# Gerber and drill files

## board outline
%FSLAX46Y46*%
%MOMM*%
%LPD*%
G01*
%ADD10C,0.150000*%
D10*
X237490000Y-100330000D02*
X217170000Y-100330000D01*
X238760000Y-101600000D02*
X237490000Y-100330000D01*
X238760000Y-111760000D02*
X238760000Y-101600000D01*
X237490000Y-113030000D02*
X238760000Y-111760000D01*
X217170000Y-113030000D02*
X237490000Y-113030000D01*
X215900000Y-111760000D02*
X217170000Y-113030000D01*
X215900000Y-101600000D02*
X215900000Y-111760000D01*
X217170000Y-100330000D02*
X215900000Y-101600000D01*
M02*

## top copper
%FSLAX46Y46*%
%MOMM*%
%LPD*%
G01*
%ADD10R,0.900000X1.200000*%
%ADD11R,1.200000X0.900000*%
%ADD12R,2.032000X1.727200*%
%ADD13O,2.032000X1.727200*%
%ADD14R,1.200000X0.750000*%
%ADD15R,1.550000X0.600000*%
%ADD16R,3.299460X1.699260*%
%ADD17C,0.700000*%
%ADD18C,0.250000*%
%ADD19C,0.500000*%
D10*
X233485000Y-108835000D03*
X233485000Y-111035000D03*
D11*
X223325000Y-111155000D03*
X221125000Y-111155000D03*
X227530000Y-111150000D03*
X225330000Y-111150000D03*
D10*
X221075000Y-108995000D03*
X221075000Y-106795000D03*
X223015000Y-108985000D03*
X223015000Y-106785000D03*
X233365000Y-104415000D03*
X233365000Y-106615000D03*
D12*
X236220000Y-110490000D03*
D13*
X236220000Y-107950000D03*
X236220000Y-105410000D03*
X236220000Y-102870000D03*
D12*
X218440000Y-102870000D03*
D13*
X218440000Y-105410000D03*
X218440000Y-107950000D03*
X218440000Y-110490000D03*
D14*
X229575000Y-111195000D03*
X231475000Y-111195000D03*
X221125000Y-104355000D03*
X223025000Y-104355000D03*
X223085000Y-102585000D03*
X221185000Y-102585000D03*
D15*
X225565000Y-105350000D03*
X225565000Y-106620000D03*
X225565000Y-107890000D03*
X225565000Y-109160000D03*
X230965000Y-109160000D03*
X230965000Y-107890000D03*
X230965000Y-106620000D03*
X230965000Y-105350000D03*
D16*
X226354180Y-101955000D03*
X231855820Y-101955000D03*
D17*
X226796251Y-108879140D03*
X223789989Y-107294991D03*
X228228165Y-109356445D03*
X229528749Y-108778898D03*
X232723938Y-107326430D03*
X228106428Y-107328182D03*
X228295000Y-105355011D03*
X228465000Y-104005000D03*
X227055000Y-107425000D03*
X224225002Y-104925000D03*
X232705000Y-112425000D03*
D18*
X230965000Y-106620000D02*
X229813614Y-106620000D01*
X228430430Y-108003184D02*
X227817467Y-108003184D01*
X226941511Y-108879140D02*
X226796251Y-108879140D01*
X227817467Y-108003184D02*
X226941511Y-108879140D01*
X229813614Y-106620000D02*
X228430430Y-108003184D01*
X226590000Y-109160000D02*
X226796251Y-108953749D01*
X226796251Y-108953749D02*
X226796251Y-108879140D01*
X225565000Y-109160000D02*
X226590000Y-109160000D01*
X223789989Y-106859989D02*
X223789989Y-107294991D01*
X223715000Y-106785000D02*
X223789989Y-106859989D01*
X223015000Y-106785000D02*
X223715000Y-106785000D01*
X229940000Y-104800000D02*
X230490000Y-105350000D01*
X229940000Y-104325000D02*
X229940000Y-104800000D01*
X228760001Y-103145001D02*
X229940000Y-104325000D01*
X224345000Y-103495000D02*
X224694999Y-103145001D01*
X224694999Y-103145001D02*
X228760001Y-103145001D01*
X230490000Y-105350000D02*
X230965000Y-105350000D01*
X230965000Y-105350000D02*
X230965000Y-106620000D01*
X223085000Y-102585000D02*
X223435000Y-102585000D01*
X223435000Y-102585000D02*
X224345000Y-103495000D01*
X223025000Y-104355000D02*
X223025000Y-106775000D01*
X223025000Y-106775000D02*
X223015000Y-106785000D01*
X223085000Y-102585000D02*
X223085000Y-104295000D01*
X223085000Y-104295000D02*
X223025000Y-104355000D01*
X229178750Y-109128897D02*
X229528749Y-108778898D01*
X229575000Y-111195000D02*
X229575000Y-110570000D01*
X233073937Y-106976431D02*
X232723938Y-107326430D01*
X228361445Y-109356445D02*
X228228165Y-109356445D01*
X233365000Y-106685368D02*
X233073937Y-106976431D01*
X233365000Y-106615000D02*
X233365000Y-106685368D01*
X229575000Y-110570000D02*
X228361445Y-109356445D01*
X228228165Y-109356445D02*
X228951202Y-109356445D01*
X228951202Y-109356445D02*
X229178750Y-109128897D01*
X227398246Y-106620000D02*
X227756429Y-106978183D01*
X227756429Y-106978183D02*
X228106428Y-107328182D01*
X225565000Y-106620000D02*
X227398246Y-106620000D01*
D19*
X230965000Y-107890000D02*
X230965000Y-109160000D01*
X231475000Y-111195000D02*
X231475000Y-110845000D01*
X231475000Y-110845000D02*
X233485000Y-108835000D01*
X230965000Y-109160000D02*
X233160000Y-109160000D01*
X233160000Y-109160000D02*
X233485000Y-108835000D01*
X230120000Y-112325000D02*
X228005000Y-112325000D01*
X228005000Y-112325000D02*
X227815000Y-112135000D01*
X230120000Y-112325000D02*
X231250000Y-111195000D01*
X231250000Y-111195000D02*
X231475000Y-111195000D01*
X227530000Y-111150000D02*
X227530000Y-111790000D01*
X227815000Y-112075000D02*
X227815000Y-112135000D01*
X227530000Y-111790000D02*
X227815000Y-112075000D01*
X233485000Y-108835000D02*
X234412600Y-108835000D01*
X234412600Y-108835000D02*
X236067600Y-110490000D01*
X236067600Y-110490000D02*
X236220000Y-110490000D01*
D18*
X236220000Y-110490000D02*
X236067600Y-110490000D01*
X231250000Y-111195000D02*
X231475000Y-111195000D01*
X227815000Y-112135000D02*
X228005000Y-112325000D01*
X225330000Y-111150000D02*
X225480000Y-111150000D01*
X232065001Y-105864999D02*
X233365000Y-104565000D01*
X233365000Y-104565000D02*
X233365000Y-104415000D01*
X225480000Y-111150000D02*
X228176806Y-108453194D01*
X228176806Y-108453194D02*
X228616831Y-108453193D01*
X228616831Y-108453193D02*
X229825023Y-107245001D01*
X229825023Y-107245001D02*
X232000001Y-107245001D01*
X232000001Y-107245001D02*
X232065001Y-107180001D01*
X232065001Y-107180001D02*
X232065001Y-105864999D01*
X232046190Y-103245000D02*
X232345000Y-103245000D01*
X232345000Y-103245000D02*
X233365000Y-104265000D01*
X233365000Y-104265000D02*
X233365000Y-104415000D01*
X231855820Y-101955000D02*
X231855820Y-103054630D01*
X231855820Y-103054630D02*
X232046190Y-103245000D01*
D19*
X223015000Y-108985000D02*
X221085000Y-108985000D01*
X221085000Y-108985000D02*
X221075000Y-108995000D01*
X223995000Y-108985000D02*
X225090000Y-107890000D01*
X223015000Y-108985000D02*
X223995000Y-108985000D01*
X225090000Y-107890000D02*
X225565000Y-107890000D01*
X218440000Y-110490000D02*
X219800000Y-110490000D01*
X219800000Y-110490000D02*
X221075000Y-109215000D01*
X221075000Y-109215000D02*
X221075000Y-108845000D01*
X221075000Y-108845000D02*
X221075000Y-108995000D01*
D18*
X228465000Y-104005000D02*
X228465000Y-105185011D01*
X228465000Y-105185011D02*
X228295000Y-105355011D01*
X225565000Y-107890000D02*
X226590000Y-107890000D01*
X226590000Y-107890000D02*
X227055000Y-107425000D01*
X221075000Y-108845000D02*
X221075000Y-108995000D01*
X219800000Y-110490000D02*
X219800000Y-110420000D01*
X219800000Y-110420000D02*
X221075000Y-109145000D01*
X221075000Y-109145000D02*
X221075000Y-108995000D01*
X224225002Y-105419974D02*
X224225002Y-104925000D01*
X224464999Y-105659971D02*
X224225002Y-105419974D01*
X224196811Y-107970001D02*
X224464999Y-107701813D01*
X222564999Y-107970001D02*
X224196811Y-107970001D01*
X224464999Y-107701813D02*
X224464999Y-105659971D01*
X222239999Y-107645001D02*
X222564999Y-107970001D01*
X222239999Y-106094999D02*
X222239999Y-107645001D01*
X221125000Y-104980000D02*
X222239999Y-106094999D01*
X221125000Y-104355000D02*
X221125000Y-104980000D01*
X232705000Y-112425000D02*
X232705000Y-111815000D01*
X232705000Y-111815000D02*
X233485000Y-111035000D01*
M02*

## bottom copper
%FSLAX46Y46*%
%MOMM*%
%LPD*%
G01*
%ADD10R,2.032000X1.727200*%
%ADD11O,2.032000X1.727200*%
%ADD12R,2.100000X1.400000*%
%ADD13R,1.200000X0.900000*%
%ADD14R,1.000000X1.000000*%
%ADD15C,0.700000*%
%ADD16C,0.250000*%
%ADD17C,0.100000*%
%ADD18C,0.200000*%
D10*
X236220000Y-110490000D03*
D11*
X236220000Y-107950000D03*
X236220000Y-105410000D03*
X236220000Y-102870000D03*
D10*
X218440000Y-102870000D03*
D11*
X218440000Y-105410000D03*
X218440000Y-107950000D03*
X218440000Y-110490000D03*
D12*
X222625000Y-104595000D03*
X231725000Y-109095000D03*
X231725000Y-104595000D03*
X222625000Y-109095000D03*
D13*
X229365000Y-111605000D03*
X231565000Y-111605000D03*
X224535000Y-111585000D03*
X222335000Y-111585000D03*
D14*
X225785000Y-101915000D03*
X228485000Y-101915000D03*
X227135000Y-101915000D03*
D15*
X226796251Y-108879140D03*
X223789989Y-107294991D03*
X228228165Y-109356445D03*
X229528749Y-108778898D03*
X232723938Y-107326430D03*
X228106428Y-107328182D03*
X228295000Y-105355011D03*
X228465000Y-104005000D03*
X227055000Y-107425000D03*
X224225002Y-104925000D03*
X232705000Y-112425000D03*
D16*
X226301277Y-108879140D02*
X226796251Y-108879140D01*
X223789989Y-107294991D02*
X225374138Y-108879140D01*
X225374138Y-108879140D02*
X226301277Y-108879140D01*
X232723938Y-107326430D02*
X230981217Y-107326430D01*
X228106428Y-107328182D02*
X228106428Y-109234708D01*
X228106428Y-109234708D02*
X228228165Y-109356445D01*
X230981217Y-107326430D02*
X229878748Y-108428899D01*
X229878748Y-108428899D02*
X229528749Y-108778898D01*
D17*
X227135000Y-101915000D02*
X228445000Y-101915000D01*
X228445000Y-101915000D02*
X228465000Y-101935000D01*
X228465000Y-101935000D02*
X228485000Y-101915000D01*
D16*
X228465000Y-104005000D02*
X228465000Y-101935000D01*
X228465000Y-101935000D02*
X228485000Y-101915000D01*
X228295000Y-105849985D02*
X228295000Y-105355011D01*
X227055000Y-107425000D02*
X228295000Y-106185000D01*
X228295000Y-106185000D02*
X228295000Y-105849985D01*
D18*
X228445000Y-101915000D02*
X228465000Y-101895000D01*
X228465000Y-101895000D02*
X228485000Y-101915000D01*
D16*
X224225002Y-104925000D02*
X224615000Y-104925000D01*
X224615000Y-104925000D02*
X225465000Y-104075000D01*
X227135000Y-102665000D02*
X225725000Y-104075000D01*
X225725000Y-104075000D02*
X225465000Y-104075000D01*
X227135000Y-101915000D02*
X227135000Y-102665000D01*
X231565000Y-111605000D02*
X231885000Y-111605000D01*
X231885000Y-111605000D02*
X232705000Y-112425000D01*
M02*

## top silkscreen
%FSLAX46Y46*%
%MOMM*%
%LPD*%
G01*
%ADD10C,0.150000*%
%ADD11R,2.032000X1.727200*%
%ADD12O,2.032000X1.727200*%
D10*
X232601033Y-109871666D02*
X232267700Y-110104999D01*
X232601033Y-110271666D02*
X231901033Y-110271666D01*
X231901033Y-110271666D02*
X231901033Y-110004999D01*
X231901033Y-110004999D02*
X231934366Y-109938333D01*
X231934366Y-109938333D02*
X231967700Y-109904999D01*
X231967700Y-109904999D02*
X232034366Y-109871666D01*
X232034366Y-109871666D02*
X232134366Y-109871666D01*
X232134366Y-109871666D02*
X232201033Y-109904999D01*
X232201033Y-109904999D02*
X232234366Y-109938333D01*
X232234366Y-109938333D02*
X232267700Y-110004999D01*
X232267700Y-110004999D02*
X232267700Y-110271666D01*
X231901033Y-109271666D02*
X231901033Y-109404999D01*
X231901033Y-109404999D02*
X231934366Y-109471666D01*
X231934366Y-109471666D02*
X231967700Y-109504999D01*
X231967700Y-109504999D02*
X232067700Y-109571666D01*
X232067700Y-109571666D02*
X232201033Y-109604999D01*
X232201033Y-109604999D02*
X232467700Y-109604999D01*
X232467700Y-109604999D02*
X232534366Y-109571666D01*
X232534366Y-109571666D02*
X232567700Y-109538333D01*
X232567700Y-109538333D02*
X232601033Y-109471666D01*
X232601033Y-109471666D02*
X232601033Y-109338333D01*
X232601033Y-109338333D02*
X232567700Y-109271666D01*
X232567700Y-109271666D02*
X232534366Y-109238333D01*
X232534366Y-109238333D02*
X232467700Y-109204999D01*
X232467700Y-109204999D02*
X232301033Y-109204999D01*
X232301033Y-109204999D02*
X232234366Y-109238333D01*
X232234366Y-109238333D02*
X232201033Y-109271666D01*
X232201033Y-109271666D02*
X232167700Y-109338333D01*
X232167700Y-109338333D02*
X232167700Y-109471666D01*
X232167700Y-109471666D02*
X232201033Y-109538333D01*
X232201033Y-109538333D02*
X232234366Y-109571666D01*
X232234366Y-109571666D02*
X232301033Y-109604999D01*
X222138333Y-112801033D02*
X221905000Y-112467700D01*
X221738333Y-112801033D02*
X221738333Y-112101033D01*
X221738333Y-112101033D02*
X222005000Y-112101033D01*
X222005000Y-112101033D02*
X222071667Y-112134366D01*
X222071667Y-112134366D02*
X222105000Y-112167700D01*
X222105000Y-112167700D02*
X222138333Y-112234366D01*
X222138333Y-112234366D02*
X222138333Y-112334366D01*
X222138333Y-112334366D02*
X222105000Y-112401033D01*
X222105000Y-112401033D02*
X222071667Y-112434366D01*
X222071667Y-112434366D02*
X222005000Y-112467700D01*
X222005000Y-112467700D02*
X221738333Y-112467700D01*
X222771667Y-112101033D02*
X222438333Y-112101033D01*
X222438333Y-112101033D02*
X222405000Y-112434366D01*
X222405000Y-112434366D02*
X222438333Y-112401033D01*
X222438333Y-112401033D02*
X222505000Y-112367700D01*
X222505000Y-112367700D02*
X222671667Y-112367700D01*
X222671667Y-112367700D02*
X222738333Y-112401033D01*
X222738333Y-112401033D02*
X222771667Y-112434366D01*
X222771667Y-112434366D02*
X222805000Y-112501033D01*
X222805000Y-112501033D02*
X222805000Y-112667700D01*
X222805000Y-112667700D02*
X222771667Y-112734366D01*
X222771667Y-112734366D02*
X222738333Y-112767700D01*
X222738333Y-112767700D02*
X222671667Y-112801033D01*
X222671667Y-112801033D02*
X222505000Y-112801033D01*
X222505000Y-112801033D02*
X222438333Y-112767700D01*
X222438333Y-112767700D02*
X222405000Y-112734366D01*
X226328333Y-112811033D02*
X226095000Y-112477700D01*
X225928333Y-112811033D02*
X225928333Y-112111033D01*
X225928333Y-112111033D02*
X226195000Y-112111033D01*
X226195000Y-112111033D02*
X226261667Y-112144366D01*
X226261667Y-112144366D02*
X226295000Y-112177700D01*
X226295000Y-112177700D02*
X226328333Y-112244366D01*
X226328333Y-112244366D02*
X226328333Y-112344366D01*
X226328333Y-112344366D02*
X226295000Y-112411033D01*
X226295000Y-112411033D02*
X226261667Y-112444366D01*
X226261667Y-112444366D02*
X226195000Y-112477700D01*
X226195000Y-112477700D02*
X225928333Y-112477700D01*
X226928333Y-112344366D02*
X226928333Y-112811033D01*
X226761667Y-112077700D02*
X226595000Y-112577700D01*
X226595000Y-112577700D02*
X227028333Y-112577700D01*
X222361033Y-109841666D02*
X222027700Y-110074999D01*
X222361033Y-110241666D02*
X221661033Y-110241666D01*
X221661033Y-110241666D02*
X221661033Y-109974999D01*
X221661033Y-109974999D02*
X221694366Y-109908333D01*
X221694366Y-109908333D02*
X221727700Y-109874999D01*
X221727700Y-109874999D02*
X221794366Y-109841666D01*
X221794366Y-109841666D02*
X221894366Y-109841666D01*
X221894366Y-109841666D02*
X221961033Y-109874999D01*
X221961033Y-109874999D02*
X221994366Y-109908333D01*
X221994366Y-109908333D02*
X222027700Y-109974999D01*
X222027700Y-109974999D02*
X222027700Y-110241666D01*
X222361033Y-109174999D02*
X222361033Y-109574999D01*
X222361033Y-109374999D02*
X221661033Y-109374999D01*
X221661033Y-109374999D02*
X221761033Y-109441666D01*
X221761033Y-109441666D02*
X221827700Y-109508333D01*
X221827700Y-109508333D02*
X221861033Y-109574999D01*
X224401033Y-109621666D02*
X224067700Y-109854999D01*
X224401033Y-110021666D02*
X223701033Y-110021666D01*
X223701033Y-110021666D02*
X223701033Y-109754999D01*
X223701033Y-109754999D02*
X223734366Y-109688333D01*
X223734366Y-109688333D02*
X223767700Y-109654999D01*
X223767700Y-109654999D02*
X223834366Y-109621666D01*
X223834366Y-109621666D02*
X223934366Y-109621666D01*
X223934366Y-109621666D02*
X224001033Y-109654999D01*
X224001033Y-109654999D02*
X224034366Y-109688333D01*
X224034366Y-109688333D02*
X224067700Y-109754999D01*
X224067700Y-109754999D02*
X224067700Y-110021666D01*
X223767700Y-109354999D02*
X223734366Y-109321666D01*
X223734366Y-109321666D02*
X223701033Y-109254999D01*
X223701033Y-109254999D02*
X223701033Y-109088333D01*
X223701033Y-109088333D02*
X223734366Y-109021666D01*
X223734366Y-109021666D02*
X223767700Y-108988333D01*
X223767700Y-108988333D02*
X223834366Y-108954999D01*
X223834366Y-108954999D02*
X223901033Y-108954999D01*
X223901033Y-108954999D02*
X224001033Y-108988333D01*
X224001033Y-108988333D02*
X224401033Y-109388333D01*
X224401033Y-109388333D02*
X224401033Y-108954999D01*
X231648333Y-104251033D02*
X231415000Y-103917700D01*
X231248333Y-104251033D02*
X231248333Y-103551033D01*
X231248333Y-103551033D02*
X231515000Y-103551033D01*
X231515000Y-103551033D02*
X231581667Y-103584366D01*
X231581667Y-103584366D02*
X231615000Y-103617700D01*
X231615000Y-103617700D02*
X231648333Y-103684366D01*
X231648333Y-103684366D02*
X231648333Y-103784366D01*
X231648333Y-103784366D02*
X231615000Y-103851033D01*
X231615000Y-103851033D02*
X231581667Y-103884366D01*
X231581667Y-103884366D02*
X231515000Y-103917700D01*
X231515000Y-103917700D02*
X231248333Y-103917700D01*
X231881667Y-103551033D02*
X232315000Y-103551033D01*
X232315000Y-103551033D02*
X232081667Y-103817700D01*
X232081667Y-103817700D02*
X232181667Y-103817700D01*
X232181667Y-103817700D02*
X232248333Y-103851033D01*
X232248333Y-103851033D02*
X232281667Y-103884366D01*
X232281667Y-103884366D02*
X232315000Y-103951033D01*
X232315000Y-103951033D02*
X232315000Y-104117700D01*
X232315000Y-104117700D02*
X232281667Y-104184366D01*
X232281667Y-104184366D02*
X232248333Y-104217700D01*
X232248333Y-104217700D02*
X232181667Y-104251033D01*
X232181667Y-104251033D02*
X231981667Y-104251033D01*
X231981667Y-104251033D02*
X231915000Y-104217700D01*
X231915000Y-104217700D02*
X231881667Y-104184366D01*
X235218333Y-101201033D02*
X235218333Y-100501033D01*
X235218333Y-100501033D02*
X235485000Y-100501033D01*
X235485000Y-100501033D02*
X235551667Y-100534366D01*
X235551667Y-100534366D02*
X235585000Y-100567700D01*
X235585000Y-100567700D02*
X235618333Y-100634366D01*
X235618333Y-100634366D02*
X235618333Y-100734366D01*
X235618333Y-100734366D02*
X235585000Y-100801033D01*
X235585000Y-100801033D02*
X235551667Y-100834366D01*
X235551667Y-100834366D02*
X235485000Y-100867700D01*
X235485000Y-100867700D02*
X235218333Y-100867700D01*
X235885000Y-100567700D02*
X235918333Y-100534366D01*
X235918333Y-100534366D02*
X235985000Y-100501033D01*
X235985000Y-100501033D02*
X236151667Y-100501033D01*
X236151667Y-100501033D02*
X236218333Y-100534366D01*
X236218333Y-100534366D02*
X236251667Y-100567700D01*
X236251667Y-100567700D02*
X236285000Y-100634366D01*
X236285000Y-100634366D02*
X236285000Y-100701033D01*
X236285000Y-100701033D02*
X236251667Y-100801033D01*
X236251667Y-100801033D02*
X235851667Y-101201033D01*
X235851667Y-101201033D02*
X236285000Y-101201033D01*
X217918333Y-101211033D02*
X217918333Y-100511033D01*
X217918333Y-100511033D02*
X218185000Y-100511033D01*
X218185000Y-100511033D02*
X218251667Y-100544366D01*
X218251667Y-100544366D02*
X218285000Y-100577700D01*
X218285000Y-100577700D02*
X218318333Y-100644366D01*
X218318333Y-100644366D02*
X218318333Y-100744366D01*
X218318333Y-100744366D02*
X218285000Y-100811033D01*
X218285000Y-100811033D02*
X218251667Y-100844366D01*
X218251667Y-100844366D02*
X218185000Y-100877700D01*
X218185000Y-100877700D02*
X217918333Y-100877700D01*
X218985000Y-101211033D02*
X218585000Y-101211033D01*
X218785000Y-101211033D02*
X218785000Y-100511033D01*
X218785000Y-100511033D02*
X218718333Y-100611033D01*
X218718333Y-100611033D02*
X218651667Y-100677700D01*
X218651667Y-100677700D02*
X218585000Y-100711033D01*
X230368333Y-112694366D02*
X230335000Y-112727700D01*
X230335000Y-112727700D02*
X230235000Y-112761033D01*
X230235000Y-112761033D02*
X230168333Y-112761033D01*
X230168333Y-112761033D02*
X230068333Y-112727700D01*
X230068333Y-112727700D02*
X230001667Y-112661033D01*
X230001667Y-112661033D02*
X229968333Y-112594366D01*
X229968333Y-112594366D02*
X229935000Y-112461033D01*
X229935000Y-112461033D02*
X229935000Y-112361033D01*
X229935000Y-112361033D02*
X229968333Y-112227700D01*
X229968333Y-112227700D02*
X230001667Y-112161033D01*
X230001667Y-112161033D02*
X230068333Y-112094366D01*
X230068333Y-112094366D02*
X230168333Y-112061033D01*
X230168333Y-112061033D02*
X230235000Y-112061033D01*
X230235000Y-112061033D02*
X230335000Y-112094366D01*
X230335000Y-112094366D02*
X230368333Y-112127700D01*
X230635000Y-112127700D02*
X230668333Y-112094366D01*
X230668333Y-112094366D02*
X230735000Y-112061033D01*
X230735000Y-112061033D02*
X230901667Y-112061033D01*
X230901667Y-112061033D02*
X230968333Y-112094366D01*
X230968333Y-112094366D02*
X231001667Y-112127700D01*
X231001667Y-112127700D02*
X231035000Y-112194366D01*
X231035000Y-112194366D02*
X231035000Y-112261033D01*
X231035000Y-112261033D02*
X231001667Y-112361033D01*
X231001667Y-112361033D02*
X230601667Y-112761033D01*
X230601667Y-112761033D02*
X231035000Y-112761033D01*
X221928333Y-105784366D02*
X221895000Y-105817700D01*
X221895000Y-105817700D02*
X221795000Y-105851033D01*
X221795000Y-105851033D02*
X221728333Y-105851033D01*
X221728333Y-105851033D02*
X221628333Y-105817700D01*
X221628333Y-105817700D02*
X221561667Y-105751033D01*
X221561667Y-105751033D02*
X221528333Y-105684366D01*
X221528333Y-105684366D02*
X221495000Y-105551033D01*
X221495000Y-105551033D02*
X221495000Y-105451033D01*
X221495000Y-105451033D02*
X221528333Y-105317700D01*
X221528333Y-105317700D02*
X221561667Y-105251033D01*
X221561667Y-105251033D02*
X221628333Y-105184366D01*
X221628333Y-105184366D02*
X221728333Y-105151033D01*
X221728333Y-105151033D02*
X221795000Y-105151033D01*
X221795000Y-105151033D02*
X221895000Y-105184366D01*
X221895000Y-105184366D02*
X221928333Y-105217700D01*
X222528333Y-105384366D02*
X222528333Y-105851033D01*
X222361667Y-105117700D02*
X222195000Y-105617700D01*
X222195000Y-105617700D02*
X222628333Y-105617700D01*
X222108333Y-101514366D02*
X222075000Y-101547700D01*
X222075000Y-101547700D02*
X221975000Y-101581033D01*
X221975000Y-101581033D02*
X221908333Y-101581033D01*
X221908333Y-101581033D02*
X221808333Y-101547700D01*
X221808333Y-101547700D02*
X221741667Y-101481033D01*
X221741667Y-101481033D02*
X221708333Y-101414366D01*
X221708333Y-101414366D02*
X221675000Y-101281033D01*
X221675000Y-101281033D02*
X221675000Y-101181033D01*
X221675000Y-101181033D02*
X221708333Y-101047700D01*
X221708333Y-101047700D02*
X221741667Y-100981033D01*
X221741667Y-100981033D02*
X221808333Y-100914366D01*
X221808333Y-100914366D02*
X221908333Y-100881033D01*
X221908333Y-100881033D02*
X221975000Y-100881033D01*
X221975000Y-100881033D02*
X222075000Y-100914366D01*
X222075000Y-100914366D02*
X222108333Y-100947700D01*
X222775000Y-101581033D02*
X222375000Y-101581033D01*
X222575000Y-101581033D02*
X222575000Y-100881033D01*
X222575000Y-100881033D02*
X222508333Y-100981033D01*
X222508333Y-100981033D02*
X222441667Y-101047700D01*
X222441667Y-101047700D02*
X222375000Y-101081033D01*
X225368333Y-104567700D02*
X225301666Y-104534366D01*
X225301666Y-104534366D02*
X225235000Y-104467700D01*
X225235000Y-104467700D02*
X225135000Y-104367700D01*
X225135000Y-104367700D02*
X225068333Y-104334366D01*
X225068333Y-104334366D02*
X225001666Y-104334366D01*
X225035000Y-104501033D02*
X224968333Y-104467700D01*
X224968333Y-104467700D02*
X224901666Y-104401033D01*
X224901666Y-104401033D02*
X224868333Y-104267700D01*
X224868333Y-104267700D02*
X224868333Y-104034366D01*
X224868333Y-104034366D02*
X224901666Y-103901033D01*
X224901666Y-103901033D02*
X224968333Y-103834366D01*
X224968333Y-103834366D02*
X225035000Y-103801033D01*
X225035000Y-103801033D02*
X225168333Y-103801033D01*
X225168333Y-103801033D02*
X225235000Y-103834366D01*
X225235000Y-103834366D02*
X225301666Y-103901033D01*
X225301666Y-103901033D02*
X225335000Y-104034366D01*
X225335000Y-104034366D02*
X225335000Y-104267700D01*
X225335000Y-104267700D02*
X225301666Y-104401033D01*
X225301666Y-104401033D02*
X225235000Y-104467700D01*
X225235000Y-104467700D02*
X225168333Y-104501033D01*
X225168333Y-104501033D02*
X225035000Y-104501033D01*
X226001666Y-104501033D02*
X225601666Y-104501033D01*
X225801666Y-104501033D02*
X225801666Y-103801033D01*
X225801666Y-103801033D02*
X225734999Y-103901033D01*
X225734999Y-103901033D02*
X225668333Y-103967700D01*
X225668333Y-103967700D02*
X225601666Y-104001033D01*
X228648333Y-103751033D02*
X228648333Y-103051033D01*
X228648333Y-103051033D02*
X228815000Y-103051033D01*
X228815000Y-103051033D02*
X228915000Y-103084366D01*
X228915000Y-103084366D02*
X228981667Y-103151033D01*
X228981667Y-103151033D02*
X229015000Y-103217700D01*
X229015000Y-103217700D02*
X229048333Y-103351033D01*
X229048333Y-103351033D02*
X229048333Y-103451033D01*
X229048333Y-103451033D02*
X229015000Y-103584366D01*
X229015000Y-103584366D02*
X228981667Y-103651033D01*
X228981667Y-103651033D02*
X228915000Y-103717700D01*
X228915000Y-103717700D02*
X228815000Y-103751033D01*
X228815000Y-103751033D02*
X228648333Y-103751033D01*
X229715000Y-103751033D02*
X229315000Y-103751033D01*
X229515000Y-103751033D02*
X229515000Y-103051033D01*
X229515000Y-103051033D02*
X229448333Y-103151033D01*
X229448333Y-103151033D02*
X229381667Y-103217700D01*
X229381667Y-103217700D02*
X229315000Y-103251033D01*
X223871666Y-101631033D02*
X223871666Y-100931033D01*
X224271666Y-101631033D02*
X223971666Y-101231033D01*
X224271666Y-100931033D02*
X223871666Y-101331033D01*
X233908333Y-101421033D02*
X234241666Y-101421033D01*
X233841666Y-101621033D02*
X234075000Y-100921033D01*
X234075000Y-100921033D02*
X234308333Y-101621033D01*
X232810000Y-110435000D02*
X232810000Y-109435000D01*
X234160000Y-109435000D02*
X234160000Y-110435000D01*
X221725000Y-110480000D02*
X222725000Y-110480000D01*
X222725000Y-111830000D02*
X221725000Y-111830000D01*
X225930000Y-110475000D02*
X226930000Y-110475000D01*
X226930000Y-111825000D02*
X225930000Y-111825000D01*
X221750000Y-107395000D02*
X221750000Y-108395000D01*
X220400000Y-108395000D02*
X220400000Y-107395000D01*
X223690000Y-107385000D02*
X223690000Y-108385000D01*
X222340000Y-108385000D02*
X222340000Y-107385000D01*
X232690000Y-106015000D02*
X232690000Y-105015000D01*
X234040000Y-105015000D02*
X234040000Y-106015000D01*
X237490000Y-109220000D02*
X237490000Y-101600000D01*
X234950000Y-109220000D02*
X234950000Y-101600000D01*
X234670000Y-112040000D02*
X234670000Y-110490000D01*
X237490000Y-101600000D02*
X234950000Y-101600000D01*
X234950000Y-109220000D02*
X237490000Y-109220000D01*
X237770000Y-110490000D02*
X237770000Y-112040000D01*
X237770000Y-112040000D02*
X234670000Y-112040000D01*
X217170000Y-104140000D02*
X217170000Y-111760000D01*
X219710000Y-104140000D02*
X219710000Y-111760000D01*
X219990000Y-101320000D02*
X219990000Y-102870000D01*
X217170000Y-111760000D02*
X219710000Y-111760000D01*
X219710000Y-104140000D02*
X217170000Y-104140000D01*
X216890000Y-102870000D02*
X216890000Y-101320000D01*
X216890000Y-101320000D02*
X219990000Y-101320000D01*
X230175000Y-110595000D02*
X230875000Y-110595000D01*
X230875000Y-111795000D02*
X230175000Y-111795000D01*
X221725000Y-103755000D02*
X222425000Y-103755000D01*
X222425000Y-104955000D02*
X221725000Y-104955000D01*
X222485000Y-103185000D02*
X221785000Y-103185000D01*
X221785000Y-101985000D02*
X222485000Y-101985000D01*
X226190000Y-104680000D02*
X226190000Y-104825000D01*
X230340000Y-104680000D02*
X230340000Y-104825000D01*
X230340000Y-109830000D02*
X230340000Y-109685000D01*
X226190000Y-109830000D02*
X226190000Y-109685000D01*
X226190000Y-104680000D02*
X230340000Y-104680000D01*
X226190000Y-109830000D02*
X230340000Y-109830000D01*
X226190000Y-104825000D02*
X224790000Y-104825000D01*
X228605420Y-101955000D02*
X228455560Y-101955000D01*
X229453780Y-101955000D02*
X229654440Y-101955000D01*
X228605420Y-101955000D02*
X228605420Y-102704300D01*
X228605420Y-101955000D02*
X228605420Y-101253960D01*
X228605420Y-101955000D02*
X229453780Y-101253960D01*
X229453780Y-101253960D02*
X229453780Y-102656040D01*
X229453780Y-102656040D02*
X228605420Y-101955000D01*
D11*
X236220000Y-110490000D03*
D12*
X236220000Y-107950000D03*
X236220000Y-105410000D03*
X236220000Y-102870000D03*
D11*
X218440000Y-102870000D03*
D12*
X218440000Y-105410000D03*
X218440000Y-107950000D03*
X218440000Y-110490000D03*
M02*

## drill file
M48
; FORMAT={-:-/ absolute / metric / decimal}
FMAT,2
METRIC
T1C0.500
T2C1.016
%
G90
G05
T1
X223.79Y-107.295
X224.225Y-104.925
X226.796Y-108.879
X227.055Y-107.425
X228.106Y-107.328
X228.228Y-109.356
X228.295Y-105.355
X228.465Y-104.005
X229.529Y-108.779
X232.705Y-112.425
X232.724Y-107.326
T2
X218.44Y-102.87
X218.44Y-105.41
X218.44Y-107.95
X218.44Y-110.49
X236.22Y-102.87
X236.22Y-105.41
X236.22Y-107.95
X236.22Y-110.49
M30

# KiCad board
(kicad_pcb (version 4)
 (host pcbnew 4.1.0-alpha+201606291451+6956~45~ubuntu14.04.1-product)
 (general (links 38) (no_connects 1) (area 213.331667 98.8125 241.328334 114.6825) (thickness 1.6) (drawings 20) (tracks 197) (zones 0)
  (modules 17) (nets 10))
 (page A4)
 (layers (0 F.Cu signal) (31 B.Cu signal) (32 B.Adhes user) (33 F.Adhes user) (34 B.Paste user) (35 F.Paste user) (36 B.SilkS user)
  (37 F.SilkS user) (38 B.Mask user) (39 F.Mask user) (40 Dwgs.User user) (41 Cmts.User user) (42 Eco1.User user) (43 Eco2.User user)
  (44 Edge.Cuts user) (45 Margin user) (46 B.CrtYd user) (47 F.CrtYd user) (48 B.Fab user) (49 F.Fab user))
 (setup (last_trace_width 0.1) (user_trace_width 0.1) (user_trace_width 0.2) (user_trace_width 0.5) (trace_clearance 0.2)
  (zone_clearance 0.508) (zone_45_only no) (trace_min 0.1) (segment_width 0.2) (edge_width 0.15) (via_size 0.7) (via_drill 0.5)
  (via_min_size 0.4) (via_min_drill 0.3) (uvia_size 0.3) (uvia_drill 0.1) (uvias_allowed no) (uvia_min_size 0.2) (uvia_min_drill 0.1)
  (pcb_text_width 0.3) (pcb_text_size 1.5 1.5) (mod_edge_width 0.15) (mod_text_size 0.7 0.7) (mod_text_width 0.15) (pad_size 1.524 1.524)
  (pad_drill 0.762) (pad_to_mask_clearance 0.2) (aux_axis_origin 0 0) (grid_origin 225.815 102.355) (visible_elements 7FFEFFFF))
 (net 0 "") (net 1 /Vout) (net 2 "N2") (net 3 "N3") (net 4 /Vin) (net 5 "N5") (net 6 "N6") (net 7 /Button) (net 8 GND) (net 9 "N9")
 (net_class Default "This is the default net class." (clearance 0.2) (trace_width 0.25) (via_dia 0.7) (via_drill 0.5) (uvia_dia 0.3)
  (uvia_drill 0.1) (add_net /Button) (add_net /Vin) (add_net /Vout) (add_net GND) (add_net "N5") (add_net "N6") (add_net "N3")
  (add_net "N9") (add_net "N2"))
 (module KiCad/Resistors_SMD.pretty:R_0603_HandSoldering (layer F.Cu) (at 233.485 109.935 270)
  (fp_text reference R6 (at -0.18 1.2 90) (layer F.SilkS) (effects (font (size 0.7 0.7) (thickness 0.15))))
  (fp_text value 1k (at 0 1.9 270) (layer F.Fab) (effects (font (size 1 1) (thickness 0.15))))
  (fp_line (start 0.5 0.675) (end -0.5 0.675) (layer F.SilkS) (width 0.15))
  (fp_line (start -0.5 -0.675) (end 0.5 -0.675) (layer F.SilkS) (width 0.15))
  (pad 1 smd rect (at -1.1 0 270) (size 1.2 0.9) (layers F.Cu F.Paste F.Mask) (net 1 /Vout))
  (pad 2 smd rect (at 1.1 0 270) (size 1.2 0.9) (layers F.Cu F.Paste F.Mask) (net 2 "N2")))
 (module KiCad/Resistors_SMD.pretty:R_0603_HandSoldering (layer F.Cu) (at 222.225 111.155 180)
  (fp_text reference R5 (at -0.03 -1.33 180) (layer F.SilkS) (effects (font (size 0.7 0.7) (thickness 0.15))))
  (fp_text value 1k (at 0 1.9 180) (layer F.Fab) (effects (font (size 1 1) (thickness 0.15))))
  (fp_line (start 0.5 0.675) (end -0.5 0.675) (layer F.SilkS) (width 0.15))
  (fp_line (start -0.5 -0.675) (end 0.5 -0.675) (layer F.SilkS) (width 0.15))
  (pad 1 smd rect (at -1.1 0 180) (size 1.2 0.9) (layers F.Cu F.Paste F.Mask))
  (pad 2 smd rect (at 1.1 0 180) (size 1.2 0.9) (layers F.Cu F.Paste F.Mask)))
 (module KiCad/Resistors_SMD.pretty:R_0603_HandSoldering (layer F.Cu) (at 226.43 111.15 180)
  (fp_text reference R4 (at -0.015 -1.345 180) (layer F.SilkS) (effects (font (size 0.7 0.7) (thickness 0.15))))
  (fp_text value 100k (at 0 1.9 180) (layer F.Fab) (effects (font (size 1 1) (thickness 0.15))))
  (fp_line (start 0.5 0.675) (end -0.5 0.675) (layer F.SilkS) (width 0.15))
  (fp_line (start -0.5 -0.675) (end 0.5 -0.675) (layer F.SilkS) (width 0.15))
  (pad 1 smd rect (at -1.1 0 180) (size 1.2 0.9) (layers F.Cu F.Paste F.Mask) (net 1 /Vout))
  (pad 2 smd rect (at 1.1 0 180) (size 1.2 0.9) (layers F.Cu F.Paste F.Mask) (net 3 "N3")))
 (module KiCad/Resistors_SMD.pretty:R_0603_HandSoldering (layer F.Cu) (at 221.075 107.895 90)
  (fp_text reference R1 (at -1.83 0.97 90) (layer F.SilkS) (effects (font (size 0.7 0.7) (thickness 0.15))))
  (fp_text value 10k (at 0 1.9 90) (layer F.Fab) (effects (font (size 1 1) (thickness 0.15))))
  (fp_line (start 0.5 0.675) (end -0.5 0.675) (layer F.SilkS) (width 0.15))
  (fp_line (start -0.5 -0.675) (end 0.5 -0.675) (layer F.SilkS) (width 0.15))
  (pad 1 smd rect (at -1.1 0 90) (size 1.2 0.9) (layers F.Cu F.Paste F.Mask) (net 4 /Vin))
  (pad 2 smd rect (at 1.1 0 90) (size 1.2 0.9) (layers F.Cu F.Paste F.Mask)))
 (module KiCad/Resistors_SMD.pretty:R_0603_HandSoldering (layer F.Cu) (at 223.015 107.885 90)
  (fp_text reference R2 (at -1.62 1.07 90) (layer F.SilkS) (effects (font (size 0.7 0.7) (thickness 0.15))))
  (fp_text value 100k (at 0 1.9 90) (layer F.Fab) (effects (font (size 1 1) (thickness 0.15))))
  (fp_line (start 0.5 0.675) (end -0.5 0.675) (layer F.SilkS) (width 0.15))
  (fp_line (start -0.5 -0.675) (end 0.5 -0.675) (layer F.SilkS) (width 0.15))
  (pad 1 smd rect (at -1.1 0 90) (size 1.2 0.9) (layers F.Cu F.Paste F.Mask) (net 4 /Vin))
  (pad 2 smd rect (at 1.1 0 90) (size 1.2 0.9) (layers F.Cu F.Paste F.Mask) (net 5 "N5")))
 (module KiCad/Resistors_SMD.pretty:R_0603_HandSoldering (layer F.Cu) (at 233.365 105.515 270)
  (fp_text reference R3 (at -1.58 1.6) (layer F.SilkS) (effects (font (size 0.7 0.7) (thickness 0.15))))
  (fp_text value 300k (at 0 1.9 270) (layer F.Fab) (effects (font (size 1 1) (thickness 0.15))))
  (fp_line (start 0.5 0.675) (end -0.5 0.675) (layer F.SilkS) (width 0.15))
  (fp_line (start -0.5 -0.675) (end 0.5 -0.675) (layer F.SilkS) (width 0.15))
  (pad 1 smd rect (at -1.1 0 270) (size 1.2 0.9) (layers F.Cu F.Paste F.Mask) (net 3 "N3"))
  (pad 2 smd rect (at 1.1 0 270) (size 1.2 0.9) (layers F.Cu F.Paste F.Mask) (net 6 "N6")))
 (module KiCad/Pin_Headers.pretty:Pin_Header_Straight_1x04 (layer F.Cu) (at 236.22 110.49 180)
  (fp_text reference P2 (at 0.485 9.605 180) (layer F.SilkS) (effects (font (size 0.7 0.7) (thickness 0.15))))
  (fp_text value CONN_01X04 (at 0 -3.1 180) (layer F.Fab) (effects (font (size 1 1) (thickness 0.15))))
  (fp_line (start -1.27 1.27) (end -1.27 8.89) (layer F.SilkS) (width 0.15))
  (fp_line (start 1.27 1.27) (end 1.27 8.89) (layer F.SilkS) (width 0.15))
  (fp_line (start 1.55 -1.55) (end 1.55 0) (layer F.SilkS) (width 0.15))
  (fp_line (start -1.27 8.89) (end 1.27 8.89) (layer F.SilkS) (width 0.15))
  (fp_line (start 1.27 1.27) (end -1.27 1.27) (layer F.SilkS) (width 0.15))
  (fp_line (start -1.55 0) (end -1.55 -1.55) (layer F.SilkS) (width 0.15))
  (fp_line (start -1.55 -1.55) (end 1.55 -1.55) (layer F.SilkS) (width 0.15))
  (pad 1 thru_hole rect (at 0 0 180) (size 2.032 1.7272) (drill 1.016) (layers *.Cu *.Mask F.SilkS) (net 1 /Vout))
  (pad 2 thru_hole oval (at 0 2.54 180) (size 2.032 1.7272) (drill 1.016) (layers *.Cu *.Mask F.SilkS))
  (pad 3 thru_hole oval (at 0 5.08 180) (size 2.032 1.7272) (drill 1.016) (layers *.Cu *.Mask F.SilkS))
  (pad 4 thru_hole oval (at 0 7.62 180) (size 2.032 1.7272) (drill 1.016) (layers *.Cu *.Mask F.SilkS)))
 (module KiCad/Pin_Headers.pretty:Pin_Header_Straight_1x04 (layer F.Cu) (at 218.44 102.87)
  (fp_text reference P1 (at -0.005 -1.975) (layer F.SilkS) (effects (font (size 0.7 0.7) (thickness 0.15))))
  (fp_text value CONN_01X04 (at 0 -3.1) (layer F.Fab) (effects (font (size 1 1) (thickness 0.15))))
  (fp_line (start -1.27 1.27) (end -1.27 8.89) (layer F.SilkS) (width 0.15))
  (fp_line (start 1.27 1.27) (end 1.27 8.89) (layer F.SilkS) (width 0.15))
  (fp_line (start 1.55 -1.55) (end 1.55 0) (layer F.SilkS) (width 0.15))
  (fp_line (start -1.27 8.89) (end 1.27 8.89) (layer F.SilkS) (width 0.15))
  (fp_line (start 1.27 1.27) (end -1.27 1.27) (layer F.SilkS) (width 0.15))
  (fp_line (start -1.55 0) (end -1.55 -1.55) (layer F.SilkS) (width 0.15))
  (fp_line (start -1.55 -1.55) (end 1.55 -1.55) (layer F.SilkS) (width 0.15))
  (pad 1 thru_hole rect (at 0 0) (size 2.032 1.7272) (drill 1.016) (layers *.Cu *.Mask F.SilkS))
  (pad 2 thru_hole oval (at 0 2.54) (size 2.032 1.7272) (drill 1.016) (layers *.Cu *.Mask F.SilkS))
  (pad 3 thru_hole oval (at 0 5.08) (size 2.032 1.7272) (drill 1.016) (layers *.Cu *.Mask F.SilkS))
  (pad 4 thru_hole oval (at 0 7.62) (size 2.032 1.7272) (drill 1.016) (layers *.Cu *.Mask F.SilkS) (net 4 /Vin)))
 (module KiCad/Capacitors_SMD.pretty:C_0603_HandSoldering (layer F.Cu) (at 230.525 111.195)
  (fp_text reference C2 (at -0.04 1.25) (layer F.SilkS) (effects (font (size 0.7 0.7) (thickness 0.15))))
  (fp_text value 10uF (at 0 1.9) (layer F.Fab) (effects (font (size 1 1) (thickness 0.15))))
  (fp_line (start -0.35 -0.6) (end 0.35 -0.6) (layer F.SilkS) (width 0.15))
  (fp_line (start 0.35 0.6) (end -0.35 0.6) (layer F.SilkS) (width 0.15))
  (pad 1 smd rect (at -0.95 0) (size 1.2 0.75) (layers F.Cu F.Paste F.Mask) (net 6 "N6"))
  (pad 2 smd rect (at 0.95 0) (size 1.2 0.75) (layers F.Cu F.Paste F.Mask) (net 1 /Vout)))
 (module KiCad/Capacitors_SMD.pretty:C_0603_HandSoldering (layer F.Cu) (at 222.075 104.355)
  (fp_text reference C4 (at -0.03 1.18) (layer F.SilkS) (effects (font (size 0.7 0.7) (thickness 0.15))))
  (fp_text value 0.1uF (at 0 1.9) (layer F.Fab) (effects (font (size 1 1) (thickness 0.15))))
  (fp_line (start -0.35 -0.6) (end 0.35 -0.6) (layer F.SilkS) (width 0.15))
  (fp_line (start 0.35 0.6) (end -0.35 0.6) (layer F.SilkS) (width 0.15))
  (pad 1 smd rect (at -0.95 0) (size 1.2 0.75) (layers F.Cu F.Paste F.Mask) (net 4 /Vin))
  (pad 2 smd rect (at 0.95 0) (size 1.2 0.75) (layers F.Cu F.Paste F.Mask) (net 5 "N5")))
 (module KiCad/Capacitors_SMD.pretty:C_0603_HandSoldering (layer F.Cu) (at 222.135 102.585 180)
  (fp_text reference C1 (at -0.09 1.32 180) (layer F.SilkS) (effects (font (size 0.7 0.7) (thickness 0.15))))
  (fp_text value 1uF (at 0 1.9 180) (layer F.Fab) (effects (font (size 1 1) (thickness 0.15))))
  (fp_line (start -0.35 -0.6) (end 0.35 -0.6) (layer F.SilkS) (width 0.15))
  (fp_line (start 0.35 0.6) (end -0.35 0.6) (layer F.SilkS) (width 0.15))
  (pad 1 smd rect (at -0.95 0 180) (size 1.2 0.75) (layers F.Cu F.Paste F.Mask) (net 5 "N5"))
  (pad 2 smd rect (at 0.95 0 180) (size 1.2 0.75) (layers F.Cu F.Paste F.Mask)))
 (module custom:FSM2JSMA (layer B.Cu) (at 227.175 106.845 270)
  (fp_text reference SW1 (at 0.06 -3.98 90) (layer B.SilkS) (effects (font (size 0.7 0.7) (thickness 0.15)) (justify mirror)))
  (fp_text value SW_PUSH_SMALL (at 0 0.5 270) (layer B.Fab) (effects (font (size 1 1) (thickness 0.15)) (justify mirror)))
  (pad 2 smd rect (at -2.25 4.55 270) (size 1.4 2.1) (layers B.Cu B.Paste B.Mask))
  (pad 1 smd rect (at 2.25 -4.55 270) (size 1.4 2.1) (layers B.Cu B.Paste B.Mask))
  (pad 2 smd rect (at -2.25 -4.55 270) (size 1.4 2.1) (layers B.Cu B.Paste B.Mask))
  (pad 1 smd rect (at 2.25 4.55 270) (size 1.4 2.1) (layers B.Cu B.Paste B.Mask)))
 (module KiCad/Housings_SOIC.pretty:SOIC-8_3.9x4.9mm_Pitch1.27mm (layer F.Cu) (at 228.265 107.255)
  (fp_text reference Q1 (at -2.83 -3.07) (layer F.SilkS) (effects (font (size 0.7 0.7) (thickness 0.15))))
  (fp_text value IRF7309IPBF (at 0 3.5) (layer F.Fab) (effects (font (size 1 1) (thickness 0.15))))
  (fp_line (start -2.075 -2.575) (end -2.075 -2.43) (layer F.SilkS) (width 0.15))
  (fp_line (start 2.075 -2.575) (end 2.075 -2.43) (layer F.SilkS) (width 0.15))
  (fp_line (start 2.075 2.575) (end 2.075 2.43) (layer F.SilkS) (width 0.15))
  (fp_line (start -2.075 2.575) (end -2.075 2.43) (layer F.SilkS) (width 0.15))
  (fp_line (start -2.075 -2.575) (end 2.075 -2.575) (layer F.SilkS) (width 0.15))
  (fp_line (start -2.075 2.575) (end 2.075 2.575) (layer F.SilkS) (width 0.15))
  (fp_line (start -2.075 -2.43) (end -3.475 -2.43) (layer F.SilkS) (width 0.15))
  (pad 1 smd rect (at -2.7 -1.905) (size 1.55 0.6) (layers F.Cu F.Paste F.Mask))
  (pad 2 smd rect (at -2.7 -0.635) (size 1.55 0.6) (layers F.Cu F.Paste F.Mask) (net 6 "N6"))
  (pad 3 smd rect (at -2.7 0.635) (size 1.55 0.6) (layers F.Cu F.Paste F.Mask) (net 4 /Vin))
  (pad 4 smd rect (at -2.7 1.905) (size 1.55 0.6) (layers F.Cu F.Paste F.Mask) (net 5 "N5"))
  (pad 5 smd rect (at 2.7 1.905) (size 1.55 0.6) (layers F.Cu F.Paste F.Mask) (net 1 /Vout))
  (pad 6 smd rect (at 2.7 0.635) (size 1.55 0.6) (layers F.Cu F.Paste F.Mask) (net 1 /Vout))
  (pad 7 smd rect (at 2.7 -0.635) (size 1.55 0.6) (layers F.Cu F.Paste F.Mask) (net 5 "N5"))
  (pad 8 smd rect (at 2.7 -1.905) (size 1.55 0.6) (layers F.Cu F.Paste F.Mask) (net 5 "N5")))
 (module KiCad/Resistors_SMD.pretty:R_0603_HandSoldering (layer B.Cu) (at 230.465 111.605)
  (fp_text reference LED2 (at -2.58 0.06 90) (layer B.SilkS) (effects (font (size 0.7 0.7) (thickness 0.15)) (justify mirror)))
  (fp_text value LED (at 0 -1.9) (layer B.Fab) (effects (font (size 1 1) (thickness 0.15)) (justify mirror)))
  (pad 1 smd rect (at -1.1 0) (size 1.2 0.9) (layers B.Cu B.Paste B.Mask))
  (pad 2 smd rect (at 1.1 0) (size 1.2 0.9) (layers B.Cu B.Paste B.Mask) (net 2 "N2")))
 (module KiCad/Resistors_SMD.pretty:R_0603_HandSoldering (layer B.Cu) (at 223.435 111.585 180)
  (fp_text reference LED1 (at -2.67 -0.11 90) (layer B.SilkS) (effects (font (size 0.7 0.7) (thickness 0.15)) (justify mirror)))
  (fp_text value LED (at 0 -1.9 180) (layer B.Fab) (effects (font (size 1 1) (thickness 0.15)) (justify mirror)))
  (pad 1 smd rect (at -1.1 0 180) (size 1.2 0.9) (layers B.Cu B.Paste B.Mask))
  (pad 2 smd rect (at 1.1 0 180) (size 1.2 0.9) (layers B.Cu B.Paste B.Mask)))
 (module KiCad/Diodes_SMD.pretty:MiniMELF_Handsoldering (layer F.Cu) (at 229.105 101.955)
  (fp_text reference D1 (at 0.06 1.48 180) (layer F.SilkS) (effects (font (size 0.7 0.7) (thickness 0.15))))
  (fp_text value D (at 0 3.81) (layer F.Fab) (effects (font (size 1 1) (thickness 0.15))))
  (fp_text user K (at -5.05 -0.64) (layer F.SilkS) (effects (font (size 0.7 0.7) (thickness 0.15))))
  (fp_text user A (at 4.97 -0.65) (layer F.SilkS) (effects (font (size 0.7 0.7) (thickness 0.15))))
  (fp_line (start -0.49958 0) (end -0.64944 0) (layer F.SilkS) (width 0.15))
  (fp_line (start 0.34878 0) (end 0.54944 0) (layer F.SilkS) (width 0.15))
  (fp_line (start -0.49958 0) (end -0.49958 0.7493) (layer F.SilkS) (width 0.15))
  (fp_line (start -0.49958 0) (end -0.49958 -0.70104) (layer F.SilkS) (width 0.15))
  (fp_line (start -0.49958 0) (end 0.34878 -0.70104) (layer F.SilkS) (width 0.15))
  (fp_line (start 0.34878 -0.70104) (end 0.34878 0.70104) (layer F.SilkS) (width 0.15))
  (fp_line (start 0.34878 0.70104) (end -0.49958 0) (layer F.SilkS) (width 0.15))
  (pad 1 smd rect (at -2.75082 0) (size 3.29946 1.69926) (layers F.Cu F.Paste F.Mask))
  (pad 2 smd rect (at 2.75082 0) (size 3.29946 1.69926) (layers F.Cu F.Paste F.Mask) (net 3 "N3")))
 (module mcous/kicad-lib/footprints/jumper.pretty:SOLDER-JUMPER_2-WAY (layer B.Cu) (at 227.135 101.915)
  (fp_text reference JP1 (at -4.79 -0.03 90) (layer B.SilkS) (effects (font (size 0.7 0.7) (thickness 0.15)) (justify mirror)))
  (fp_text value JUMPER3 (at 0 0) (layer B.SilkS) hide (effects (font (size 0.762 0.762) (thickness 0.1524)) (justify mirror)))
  (pad 1 smd rect (at -1.35 0) (size 1 1) (layers B.Cu B.Paste B.Mask))
  (pad 3 smd rect (at 1.35 0) (size 1 1) (layers B.Cu B.Paste B.Mask) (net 4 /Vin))
  (pad 2 smd rect (at 0 0) (size 1 1) (layers B.Cu B.Paste B.Mask) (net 4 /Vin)))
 (gr_line (start 237.49 100.33) (end 217.17 100.33) (angle 90) (layer Edge.Cuts) (width 0.15))
 (gr_line (start 238.76 101.6) (end 237.49 100.33) (angle 90) (layer Edge.Cuts) (width 0.15))
 (gr_line (start 238.76 111.76) (end 238.76 101.6) (angle 90) (layer Edge.Cuts) (width 0.15))
 (gr_line (start 237.49 113.03) (end 238.76 111.76) (angle 90) (layer Edge.Cuts) (width 0.15))
 (gr_line (start 217.17 113.03) (end 237.49 113.03) (angle 90) (layer Edge.Cuts) (width 0.15))
 (gr_line (start 215.9 111.76) (end 217.17 113.03) (angle 90) (layer Edge.Cuts) (width 0.15))
 (gr_line (start 215.9 101.6) (end 215.9 111.76) (angle 90) (layer Edge.Cuts) (width 0.15))
 (gr_line (start 217.17 100.33) (end 215.9 101.6) (angle 90) (layer Edge.Cuts) (width 0.15))
 (segment (start 230.965 106.62) (end 229.813614 106.62) (width 0.25) (layer F.Cu) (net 5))
 (segment (start 228.43043 108.003184) (end 227.817467 108.003184) (width 0.25) (layer F.Cu) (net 5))
 (segment (start 226.941511 108.87914) (end 226.796251 108.87914) (width 0.25) (layer F.Cu) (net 5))
 (segment (start 227.817467 108.003184) (end 226.941511 108.87914) (width 0.25) (layer F.Cu) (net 5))
 (segment (start 226.301277 108.87914) (end 226.796251 108.87914) (width 0.25) (layer B.Cu) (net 5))
 (segment (start 229.813614 106.62) (end 228.43043 108.003184) (width 0.25) (layer F.Cu) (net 5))
 (segment (start 223.789989 107.294991) (end 225.374138 108.87914) (width 0.25) (layer B.Cu) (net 5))
 (segment (start 226.59 109.16) (end 226.796251 108.953749) (width 0.25) (layer F.Cu) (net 5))
 (segment (start 225.374138 108.87914) (end 226.301277 108.87914) (width 0.25) (layer B.Cu) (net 5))
 (segment (start 226.796251 108.953749) (end 226.796251 108.87914) (width 0.25) (layer F.Cu) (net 5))
 (segment (start 225.565 109.16) (end 226.59 109.16) (width 0.25) (layer F.Cu) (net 5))
 (segment (start 223.789989 106.859989) (end 223.789989 107.294991) (width 0.25) (layer F.Cu) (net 5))
 (segment (start 223.715 106.785) (end 223.789989 106.859989) (width 0.25) (layer F.Cu) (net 5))
 (segment (start 223.015 106.785) (end 223.715 106.785) (width 0.25) (layer F.Cu) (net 5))
 (segment (start 229.94 104.8) (end 230.49 105.35) (width 0.25) (layer F.Cu) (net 5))
 (segment (start 229.94 104.325) (end 229.94 104.8) (width 0.25) (layer F.Cu) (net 5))
 (segment (start 228.760001 103.145001) (end 229.94 104.325) (width 0.25) (layer F.Cu) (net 5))
 (segment (start 224.345 103.495) (end 224.694999 103.145001) (width 0.25) (layer F.Cu) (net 5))
 (segment (start 224.694999 103.145001) (end 228.760001 103.145001) (width 0.25) (layer F.Cu) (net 5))
 (segment (start 230.49 105.35) (end 230.965 105.35) (width 0.25) (layer F.Cu) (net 5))
 (segment (start 230.965 105.35) (end 230.965 106.62) (width 0.25) (layer F.Cu) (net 5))
 (segment (start 223.085 102.585) (end 223.435 102.585) (width 0.25) (layer F.Cu) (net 5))
 (segment (start 223.435 102.585) (end 224.345 103.495) (width 0.25) (layer F.Cu) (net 5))
 (segment (start 223.025 104.355) (end 223.025 106.775) (width 0.25) (layer F.Cu) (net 5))
 (segment (start 223.025 106.775) (end 223.015 106.785) (width 0.25) (layer F.Cu) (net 5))
 (segment (start 223.085 102.585) (end 223.085 104.295) (width 0.25) (layer F.Cu) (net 5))
 (segment (start 223.085 104.295) (end 223.025 104.355) (width 0.25) (layer F.Cu) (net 5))
 (segment (start 229.17875 109.128897) (end 229.528749 108.778898) (width 0.25) (layer F.Cu) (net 6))
 (segment (start 229.575 111.195) (end 229.575 110.57) (width 0.25) (layer F.Cu) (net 6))
 (segment (start 233.073937 106.976431) (end 232.723938 107.32643) (width 0.25) (layer F.Cu) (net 6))
 (segment (start 232.723938 107.32643) (end 230.981217 107.32643) (width 0.25) (layer B.Cu) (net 6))
 (segment (start 228.361445 109.356445) (end 228.228165 109.356445) (width 0.25) (layer F.Cu) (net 6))
 (segment (start 233.365 106.685368) (end 233.073937 106.976431) (width 0.25) (layer F.Cu) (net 6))
 (segment (start 228.106428 107.328182) (end 228.106428 109.234708) (width 0.25) (layer B.Cu) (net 6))
 (segment (start 228.106428 109.234708) (end 228.228165 109.356445) (width 0.25) (layer B.Cu) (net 6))
 (segment (start 233.365 106.615) (end 233.365 106.685368) (width 0.25) (layer F.Cu) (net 6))
 (segment (start 229.575 110.57) (end 228.361445 109.356445) (width 0.25) (layer F.Cu) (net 6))
 (segment (start 230.981217 107.32643) (end 229.878748 108.428899) (width 0.25) (layer B.Cu) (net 6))
 (segment (start 229.878748 108.428899) (end 229.528749 108.778898) (width 0.25) (layer B.Cu) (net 6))
 (segment (start 228.228165 109.356445) (end 228.951202 109.356445) (width 0.25) (layer F.Cu) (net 6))
 (segment (start 228.951202 109.356445) (end 229.17875 109.128897) (width 0.25) (layer F.Cu) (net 6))
 (segment (start 227.398246 106.62) (end 227.756429 106.978183) (width 0.25) (layer F.Cu) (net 6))
 (segment (start 227.756429 106.978183) (end 228.106428 107.328182) (width 0.25) (layer F.Cu) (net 6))
 (segment (start 225.565 106.62) (end 227.398246 106.62) (width 0.25) (layer F.Cu) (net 6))
 (segment (start 230.965 107.89) (end 230.965 109.16) (width 0.5) (layer F.Cu) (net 1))
 (segment (start 231.475 111.195) (end 231.475 110.845) (width 0.5) (layer F.Cu) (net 1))
 (segment (start 231.475 110.845) (end 233.485 108.835) (width 0.5) (layer F.Cu) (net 1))
 (segment (start 230.965 109.16) (end 233.16 109.16) (width 0.5) (layer F.Cu) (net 1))
 (segment (start 233.16 109.16) (end 233.485 108.835) (width 0.5) (layer F.Cu) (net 1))
 (segment (start 230.12 112.325) (end 228.005 112.325) (width 0.5) (layer F.Cu) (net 1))
 (segment (start 228.005 112.325) (end 227.815 112.135) (width 0.5) (layer F.Cu) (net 1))
 (segment (start 230.12 112.325) (end 231.25 111.195) (width 0.5) (layer F.Cu) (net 1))
 (segment (start 231.25 111.195) (end 231.475 111.195) (width 0.5) (layer F.Cu) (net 1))
 (segment (start 227.53 111.15) (end 227.53 111.79) (width 0.5) (layer F.Cu) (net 1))
 (segment (start 227.815 112.075) (end 227.815 112.135) (width 0.5) (layer F.Cu) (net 1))
 (segment (start 227.53 111.79) (end 227.815 112.075) (width 0.5) (layer F.Cu) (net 1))
 (segment (start 233.485 108.835) (end 234.4126 108.835) (width 0.5) (layer F.Cu) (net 1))
 (segment (start 234.4126 108.835) (end 236.0676 110.49) (width 0.5) (layer F.Cu) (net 1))
 (segment (start 236.0676 110.49) (end 236.22 110.49) (width 0.5) (layer F.Cu) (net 1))
 (segment (start 236.22 110.49) (end 236.0676 110.49) (width 0.25) (layer F.Cu) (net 1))
 (segment (start 231.25 111.195) (end 231.475 111.195) (width 0.25) (layer F.Cu) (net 1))
 (segment (start 227.815 112.135) (end 228.005 112.325) (width 0.25) (layer F.Cu) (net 1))
 (segment (start 225.33 111.15) (end 225.48 111.15) (width 0.25) (layer F.Cu) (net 3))
 (segment (start 232.065001 105.864999) (end 233.365 104.565) (width 0.25) (layer F.Cu) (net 3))
 (segment (start 233.365 104.565) (end 233.365 104.415) (width 0.25) (layer F.Cu) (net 3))
 (segment (start 225.48 111.15) (end 228.176806 108.453194) (width 0.25) (layer F.Cu) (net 3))
 (segment (start 228.176806 108.453194) (end 228.616831 108.453193) (width 0.25) (layer F.Cu) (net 3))
 (segment (start 228.616831 108.453193) (end 229.825023 107.245001) (width 0.25) (layer F.Cu) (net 3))
 (segment (start 229.825023 107.245001) (end 232.000001 107.245001) (width 0.25) (layer F.Cu) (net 3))
 (segment (start 232.000001 107.245001) (end 232.065001 107.180001) (width 0.25) (layer F.Cu) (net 3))
 (segment (start 232.065001 107.180001) (end 232.065001 105.864999) (width 0.25) (layer F.Cu) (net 3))
 (segment (start 232.04619 103.245) (end 232.345 103.245) (width 0.25) (layer F.Cu) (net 3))
 (segment (start 232.345 103.245) (end 233.365 104.265) (width 0.25) (layer F.Cu) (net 3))
 (segment (start 233.365 104.265) (end 233.365 104.415) (width 0.25) (layer F.Cu) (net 3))
 (segment (start 231.85582 101.955) (end 231.85582 103.05463) (width 0.25) (layer F.Cu) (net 3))
 (segment (start 231.85582 103.05463) (end 232.04619 103.245) (width 0.25) (layer F.Cu) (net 3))
 (segment (start 227.135 101.915) (end 228.445 101.915) (width 0.1) (layer B.Cu) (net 4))
 (segment (start 228.445 101.915) (end 228.465 101.935) (width 0.1) (layer B.Cu) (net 4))
 (segment (start 228.465 101.935) (end 228.485 101.915) (width 0.1) (layer B.Cu) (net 4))
 (segment (start 223.015 108.985) (end 221.085 108.985) (width 0.5) (layer F.Cu) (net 4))
 (segment (start 221.085 108.985) (end 221.075 108.995) (width 0.5) (layer F.Cu) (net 4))
 (segment (start 223.995 108.985) (end 225.09 107.89) (width 0.5) (layer F.Cu) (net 4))
 (segment (start 223.015 108.985) (end 223.995 108.985) (width 0.5) (layer F.Cu) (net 4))
 (segment (start 225.09 107.89) (end 225.565 107.89) (width 0.5) (layer F.Cu) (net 4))
 (segment (start 218.44 110.49) (end 219.8 110.49) (width 0.5) (layer F.Cu) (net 4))
 (segment (start 219.8 110.49) (end 221.075 109.215) (width 0.5) (layer F.Cu) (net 4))
 (segment (start 221.075 109.215) (end 221.075 108.845) (width 0.5) (layer F.Cu) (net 4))
 (segment (start 221.075 108.845) (end 221.075 108.995) (width 0.5) (layer F.Cu) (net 4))
 (segment (start 228.465 104.005) (end 228.465 101.935) (width 0.25) (layer B.Cu) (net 4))
 (segment (start 228.465 101.935) (end 228.485 101.915) (width 0.25) (layer B.Cu) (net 4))
 (segment (start 228.465 104.005) (end 228.465 105.185011) (width 0.25) (layer F.Cu) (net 4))
 (segment (start 228.295 105.849985) (end 228.295 105.355011) (width 0.25) (layer B.Cu) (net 4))
 (segment (start 227.055 107.425) (end 228.295 106.185) (width 0.25) (layer B.Cu) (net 4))
 (segment (start 228.465 105.185011) (end 228.295 105.355011) (width 0.25) (layer F.Cu) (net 4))
 (segment (start 228.295 106.185) (end 228.295 105.849985) (width 0.25) (layer B.Cu) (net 4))
 (segment (start 225.565 107.89) (end 226.59 107.89) (width 0.25) (layer F.Cu) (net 4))
 (segment (start 226.59 107.89) (end 227.055 107.425) (width 0.25) (layer F.Cu) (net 4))
 (segment (start 228.445 101.915) (end 228.465 101.895) (width 0.2) (layer B.Cu) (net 4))
 (segment (start 228.465 101.895) (end 228.485 101.915) (width 0.2) (layer B.Cu) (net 4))
 (segment (start 221.075 108.845) (end 221.075 108.995) (width 0.25) (layer F.Cu) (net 4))
 (segment (start 219.8 110.49) (end 219.8 110.42) (width 0.25) (layer F.Cu) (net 4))
 (segment (start 219.8 110.42) (end 221.075 109.145) (width 0.25) (layer F.Cu) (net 4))
 (segment (start 221.075 109.145) (end 221.075 108.995) (width 0.25) (layer F.Cu) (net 4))
 (segment (start 224.225002 105.419974) (end 224.225002 104.925) (width 0.25) (layer F.Cu) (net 4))
 (segment (start 224.464999 105.659971) (end 224.225002 105.419974) (width 0.25) (layer F.Cu) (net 4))
 (segment (start 224.196811 107.970001) (end 224.464999 107.701813) (width 0.25) (layer F.Cu) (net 4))
 (segment (start 222.564999 107.970001) (end 224.196811 107.970001) (width 0.25) (layer F.Cu) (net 4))
 (segment (start 224.464999 107.701813) (end 224.464999 105.659971) (width 0.25) (layer F.Cu) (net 4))
 (segment (start 222.239999 107.645001) (end 222.564999 107.970001) (width 0.25) (layer F.Cu) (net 4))
 (segment (start 222.239999 106.094999) (end 222.239999 107.645001) (width 0.25) (layer F.Cu) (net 4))
 (segment (start 221.125 104.98) (end 222.239999 106.094999) (width 0.25) (layer F.Cu) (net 4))
 (segment (start 221.125 104.355) (end 221.125 104.98) (width 0.25) (layer F.Cu) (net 4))
 (segment (start 224.225002 104.925) (end 224.615 104.925) (width 0.25) (layer B.Cu) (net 4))
 (segment (start 224.615 104.925) (end 225.465 104.075) (width 0.25) (layer B.Cu) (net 4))
 (segment (start 227.135 102.665) (end 225.725 104.075) (width 0.25) (layer B.Cu) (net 4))
 (segment (start 225.725 104.075) (end 225.465 104.075) (width 0.25) (layer B.Cu) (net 4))
 (segment (start 227.135 101.915) (end 227.135 102.665) (width 0.25) (layer B.Cu) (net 4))
 (segment (start 232.705 112.425) (end 232.705 111.815) (width 0.25) (layer F.Cu) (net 2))
 (segment (start 232.705 111.815) (end 233.485 111.035) (width 0.25) (layer F.Cu) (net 2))
 (segment (start 231.565 111.605) (end 231.885 111.605) (width 0.25) (layer B.Cu) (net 2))
 (segment (start 231.885 111.605) (end 232.705 112.425) (width 0.25) (layer B.Cu) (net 2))
 (via (at 226.796251 108.87914) (size 0.7) (layers F.Cu B.Cu) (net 5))
 (via (at 223.789989 107.294991) (size 0.7) (layers F.Cu B.Cu) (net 5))
 (via (at 228.228165 109.356445) (size 0.7) (layers F.Cu B.Cu) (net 6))
 (via (at 229.528749 108.778898) (size 0.7) (layers F.Cu B.Cu) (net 6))
 (via (at 232.723938 107.32643) (size 0.7) (layers F.Cu B.Cu) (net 6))
 (via (at 228.106428 107.328182) (size 0.7) (layers F.Cu B.Cu) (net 6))
 (via (at 228.295 105.355011) (size 0.7) (layers F.Cu B.Cu) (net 4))
 (via (at 228.465 104.005) (size 0.7) (layers F.Cu B.Cu) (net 4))
 (via (at 227.055 107.425) (size 0.7) (layers F.Cu B.Cu) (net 4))
 (via (at 224.225002 104.925) (size 0.7) (layers F.Cu B.Cu) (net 4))
 (via (at 232.705 112.425) (size 0.7) (layers F.Cu B.Cu) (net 2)))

